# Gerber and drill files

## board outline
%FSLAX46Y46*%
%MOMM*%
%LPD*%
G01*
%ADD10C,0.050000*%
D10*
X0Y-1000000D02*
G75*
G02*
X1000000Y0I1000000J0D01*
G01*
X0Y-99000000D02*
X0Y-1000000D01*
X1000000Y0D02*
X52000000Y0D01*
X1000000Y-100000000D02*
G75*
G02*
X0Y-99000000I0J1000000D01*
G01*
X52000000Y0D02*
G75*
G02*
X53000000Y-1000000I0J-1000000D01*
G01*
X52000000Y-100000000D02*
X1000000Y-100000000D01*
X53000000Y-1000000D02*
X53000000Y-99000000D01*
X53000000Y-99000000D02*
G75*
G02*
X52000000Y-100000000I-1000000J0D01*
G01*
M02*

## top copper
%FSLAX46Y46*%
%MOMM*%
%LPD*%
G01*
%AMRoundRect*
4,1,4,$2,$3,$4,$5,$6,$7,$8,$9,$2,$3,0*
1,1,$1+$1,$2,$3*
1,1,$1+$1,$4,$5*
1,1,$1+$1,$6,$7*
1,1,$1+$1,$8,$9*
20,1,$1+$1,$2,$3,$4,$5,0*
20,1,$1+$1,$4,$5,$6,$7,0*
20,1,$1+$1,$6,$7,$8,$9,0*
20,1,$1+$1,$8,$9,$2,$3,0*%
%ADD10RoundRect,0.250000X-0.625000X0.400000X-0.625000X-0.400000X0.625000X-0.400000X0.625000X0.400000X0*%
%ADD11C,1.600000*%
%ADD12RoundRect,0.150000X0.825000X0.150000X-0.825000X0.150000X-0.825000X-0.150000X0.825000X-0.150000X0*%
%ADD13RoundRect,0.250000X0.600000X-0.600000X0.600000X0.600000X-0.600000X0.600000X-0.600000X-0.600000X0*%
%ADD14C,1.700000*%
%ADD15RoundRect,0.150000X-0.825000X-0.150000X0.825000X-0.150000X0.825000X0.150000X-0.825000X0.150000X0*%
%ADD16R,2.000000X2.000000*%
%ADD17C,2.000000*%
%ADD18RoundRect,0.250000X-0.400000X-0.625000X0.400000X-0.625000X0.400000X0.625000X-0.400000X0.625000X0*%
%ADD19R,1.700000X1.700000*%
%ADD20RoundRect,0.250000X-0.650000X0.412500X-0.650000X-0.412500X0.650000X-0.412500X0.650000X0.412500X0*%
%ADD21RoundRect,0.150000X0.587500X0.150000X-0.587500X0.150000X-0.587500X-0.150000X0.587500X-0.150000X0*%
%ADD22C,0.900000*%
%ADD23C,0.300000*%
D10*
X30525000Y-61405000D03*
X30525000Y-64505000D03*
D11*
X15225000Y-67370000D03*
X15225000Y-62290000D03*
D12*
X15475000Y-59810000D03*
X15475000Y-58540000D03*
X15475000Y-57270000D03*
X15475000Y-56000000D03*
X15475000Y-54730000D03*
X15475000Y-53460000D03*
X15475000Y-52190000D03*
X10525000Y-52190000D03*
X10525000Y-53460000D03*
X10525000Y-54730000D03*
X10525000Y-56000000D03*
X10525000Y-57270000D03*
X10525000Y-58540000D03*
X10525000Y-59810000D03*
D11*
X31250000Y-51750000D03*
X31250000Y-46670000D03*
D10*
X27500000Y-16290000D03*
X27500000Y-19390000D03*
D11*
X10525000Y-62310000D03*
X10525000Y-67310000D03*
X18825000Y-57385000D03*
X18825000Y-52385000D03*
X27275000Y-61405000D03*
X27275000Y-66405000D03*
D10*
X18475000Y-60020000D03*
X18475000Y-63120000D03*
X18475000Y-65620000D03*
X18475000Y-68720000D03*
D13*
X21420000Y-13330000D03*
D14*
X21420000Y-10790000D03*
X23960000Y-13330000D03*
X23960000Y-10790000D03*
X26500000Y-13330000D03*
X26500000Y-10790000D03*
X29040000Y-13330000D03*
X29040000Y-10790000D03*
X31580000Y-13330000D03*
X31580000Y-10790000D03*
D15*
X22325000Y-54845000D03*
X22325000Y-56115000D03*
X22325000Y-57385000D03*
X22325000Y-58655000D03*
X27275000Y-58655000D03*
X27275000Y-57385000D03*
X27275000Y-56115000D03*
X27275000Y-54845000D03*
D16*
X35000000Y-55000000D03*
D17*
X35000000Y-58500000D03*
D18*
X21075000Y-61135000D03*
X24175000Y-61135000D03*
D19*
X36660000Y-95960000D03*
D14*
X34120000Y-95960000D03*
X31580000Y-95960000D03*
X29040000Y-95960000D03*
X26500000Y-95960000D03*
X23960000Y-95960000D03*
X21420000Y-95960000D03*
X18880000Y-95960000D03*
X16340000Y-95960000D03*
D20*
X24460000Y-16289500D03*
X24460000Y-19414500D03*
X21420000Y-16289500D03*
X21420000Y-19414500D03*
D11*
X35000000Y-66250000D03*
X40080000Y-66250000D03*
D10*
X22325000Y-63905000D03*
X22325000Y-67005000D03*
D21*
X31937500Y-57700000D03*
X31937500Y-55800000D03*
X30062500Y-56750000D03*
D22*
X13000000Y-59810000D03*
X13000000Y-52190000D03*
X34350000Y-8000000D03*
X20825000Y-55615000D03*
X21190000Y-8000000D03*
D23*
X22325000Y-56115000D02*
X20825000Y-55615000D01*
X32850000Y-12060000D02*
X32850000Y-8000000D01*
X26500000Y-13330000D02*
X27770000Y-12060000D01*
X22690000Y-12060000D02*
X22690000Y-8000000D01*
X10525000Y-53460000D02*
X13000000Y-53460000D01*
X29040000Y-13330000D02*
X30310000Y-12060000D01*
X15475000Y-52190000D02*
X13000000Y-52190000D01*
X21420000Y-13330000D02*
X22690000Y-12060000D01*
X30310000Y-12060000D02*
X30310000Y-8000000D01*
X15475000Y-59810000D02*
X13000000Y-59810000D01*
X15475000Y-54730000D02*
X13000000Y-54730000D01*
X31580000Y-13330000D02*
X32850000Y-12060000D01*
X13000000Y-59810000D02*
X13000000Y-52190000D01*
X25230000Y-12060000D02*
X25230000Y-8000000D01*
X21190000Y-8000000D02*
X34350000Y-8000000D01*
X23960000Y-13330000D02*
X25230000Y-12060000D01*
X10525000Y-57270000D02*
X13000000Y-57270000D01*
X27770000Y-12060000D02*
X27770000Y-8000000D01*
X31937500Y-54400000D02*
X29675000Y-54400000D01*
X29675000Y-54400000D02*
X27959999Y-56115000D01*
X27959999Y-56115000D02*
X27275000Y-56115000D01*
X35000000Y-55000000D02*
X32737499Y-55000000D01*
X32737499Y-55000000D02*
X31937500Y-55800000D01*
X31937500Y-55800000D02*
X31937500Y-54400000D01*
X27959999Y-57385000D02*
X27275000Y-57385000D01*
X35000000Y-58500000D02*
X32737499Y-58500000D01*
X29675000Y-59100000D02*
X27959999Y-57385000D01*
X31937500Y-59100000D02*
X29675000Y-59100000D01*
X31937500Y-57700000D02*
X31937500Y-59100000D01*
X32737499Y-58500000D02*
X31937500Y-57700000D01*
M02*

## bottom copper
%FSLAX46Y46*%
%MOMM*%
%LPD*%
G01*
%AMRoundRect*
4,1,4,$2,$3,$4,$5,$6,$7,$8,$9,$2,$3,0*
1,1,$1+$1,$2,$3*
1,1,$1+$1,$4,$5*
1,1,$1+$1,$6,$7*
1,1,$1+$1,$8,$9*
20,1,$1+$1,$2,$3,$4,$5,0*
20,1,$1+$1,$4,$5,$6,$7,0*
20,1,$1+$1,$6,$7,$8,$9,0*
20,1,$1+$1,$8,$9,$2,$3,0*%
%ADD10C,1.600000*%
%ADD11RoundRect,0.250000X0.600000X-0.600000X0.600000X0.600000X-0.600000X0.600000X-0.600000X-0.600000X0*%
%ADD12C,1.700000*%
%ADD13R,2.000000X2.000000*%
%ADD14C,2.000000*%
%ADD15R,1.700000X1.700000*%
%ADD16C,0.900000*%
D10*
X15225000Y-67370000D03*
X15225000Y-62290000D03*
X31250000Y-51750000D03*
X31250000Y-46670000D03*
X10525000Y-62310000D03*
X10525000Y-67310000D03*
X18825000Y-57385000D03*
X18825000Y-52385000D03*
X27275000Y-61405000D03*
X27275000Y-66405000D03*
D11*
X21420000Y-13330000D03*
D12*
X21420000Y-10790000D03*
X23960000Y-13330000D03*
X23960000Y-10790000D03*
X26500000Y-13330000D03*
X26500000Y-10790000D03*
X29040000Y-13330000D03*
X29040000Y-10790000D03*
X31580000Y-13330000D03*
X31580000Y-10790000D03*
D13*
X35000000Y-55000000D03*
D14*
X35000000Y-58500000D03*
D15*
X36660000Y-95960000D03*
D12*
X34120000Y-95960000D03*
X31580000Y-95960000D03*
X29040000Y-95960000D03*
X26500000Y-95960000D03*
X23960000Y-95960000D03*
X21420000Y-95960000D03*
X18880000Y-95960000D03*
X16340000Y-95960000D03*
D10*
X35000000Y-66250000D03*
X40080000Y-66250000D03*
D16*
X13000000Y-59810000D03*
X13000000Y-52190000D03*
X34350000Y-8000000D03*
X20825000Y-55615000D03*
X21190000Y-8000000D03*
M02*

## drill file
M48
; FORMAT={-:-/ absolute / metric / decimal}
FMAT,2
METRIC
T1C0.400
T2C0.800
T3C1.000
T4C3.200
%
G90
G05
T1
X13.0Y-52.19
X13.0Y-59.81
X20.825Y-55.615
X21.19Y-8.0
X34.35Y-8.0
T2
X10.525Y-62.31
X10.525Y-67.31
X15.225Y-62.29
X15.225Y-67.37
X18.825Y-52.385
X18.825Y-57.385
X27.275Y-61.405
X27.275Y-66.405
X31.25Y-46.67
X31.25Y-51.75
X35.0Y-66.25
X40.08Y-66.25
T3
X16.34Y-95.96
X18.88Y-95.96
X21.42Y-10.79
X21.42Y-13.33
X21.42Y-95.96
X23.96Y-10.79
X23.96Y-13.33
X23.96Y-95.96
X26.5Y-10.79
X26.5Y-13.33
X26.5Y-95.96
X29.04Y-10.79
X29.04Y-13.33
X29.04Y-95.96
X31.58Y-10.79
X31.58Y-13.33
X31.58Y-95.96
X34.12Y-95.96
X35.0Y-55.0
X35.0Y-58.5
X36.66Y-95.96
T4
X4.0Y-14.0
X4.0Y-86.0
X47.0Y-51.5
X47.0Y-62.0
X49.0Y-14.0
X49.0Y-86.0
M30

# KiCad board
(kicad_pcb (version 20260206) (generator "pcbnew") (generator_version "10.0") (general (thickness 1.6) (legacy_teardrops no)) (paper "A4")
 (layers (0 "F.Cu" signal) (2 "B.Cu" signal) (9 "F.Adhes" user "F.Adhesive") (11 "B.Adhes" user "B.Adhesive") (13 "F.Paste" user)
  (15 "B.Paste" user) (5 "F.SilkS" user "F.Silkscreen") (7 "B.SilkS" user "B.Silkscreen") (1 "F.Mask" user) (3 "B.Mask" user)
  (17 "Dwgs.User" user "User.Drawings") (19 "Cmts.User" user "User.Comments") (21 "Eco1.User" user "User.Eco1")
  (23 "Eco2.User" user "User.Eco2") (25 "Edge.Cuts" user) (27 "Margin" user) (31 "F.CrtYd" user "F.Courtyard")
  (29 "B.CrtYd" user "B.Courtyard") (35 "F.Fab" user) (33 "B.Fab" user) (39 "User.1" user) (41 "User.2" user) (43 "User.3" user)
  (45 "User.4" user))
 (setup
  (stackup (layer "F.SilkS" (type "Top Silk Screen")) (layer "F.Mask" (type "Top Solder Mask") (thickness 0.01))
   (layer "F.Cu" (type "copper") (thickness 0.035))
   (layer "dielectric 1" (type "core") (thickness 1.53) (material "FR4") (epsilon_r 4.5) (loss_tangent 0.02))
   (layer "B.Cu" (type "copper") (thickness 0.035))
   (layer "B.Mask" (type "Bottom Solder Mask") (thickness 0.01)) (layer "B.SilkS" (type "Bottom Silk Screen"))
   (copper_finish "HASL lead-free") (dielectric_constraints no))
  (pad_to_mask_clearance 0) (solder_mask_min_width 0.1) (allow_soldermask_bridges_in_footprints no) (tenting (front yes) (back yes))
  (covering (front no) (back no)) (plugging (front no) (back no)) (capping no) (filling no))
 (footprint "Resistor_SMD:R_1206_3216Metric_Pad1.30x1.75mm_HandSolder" (layer "F.Cu") (at 30.525 62.955 -90)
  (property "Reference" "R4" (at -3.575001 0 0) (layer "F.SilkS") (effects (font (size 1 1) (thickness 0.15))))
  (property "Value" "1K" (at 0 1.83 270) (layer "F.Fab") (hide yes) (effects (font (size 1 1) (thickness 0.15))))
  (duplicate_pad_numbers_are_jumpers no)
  (pad "1" smd roundrect (at -1.55 0 270) (size 1.3 1.75) (layers "F.Cu" "F.Mask" "F.Paste") (roundrect_rratio 0.192308) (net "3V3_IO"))
  (pad "2" smd roundrect (at 1.55 0 270) (size 1.3 1.75) (layers "F.Cu" "F.Mask" "F.Paste") (roundrect_rratio 0.192308)
   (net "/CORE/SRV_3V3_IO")))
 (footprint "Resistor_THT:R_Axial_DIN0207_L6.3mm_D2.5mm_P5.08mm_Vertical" (layer "F.Cu") (at 15.225 67.37 90)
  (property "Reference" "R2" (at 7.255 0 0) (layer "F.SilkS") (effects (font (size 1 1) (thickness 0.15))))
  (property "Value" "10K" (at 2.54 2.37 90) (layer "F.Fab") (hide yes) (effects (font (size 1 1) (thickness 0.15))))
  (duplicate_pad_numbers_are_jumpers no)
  (pad "1" thru_hole circle (at 0 0 90) (size 1.6 1.6) (drill 0.8) (layers "*.Cu" "*.Mask") (remove_unused_layers no) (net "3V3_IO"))
  (pad "2" thru_hole circle (at 5.08 0 90) (size 1.6 1.6) (drill 0.8) (layers "*.Cu" "*.Mask") (remove_unused_layers no) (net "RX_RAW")))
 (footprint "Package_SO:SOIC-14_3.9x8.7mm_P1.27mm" (layer "F.Cu") (at 13 56 180)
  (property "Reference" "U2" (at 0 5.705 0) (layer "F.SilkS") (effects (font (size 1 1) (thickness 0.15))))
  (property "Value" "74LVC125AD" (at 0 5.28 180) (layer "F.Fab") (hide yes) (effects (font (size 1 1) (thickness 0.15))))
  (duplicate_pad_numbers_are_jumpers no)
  (pad "1" smd roundrect (at -2.475 -3.81 180) (size 1.95 0.6) (layers "F.Cu" "F.Mask" "F.Paste") (roundrect_rratio 0.25) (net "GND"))
  (pad "2" smd roundrect (at -2.475 -2.54 180) (size 1.95 0.6) (layers "F.Cu" "F.Mask" "F.Paste") (roundrect_rratio 0.25) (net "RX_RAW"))
  (pad "3" smd roundrect (at -2.475 -1.27 180) (size 1.95 0.6) (layers "F.Cu" "F.Mask" "F.Paste") (roundrect_rratio 0.25)
   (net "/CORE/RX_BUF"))
  (pad "4" smd roundrect (at -2.475 0 180) (size 1.95 0.6) (layers "F.Cu" "F.Mask" "F.Paste") (roundrect_rratio 0.25) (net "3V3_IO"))
  (pad "5" smd roundrect (at -2.475 1.27 180) (size 1.95 0.6) (layers "F.Cu" "F.Mask" "F.Paste") (roundrect_rratio 0.25) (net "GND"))
  (pad "6" smd roundrect (at -2.475 2.54 180) (size 1.95 0.6) (layers "F.Cu" "F.Mask" "F.Paste") (roundrect_rratio 0.25)
   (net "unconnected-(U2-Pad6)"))
  (pad "7" smd roundrect (at -2.475 3.81 180) (size 1.95 0.6) (layers "F.Cu" "F.Mask" "F.Paste") (roundrect_rratio 0.25) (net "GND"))
  (pad "8" smd roundrect (at 2.475 3.81 180) (size 1.95 0.6) (layers "F.Cu" "F.Mask" "F.Paste") (roundrect_rratio 0.25)
   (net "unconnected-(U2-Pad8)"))
  (pad "9" smd roundrect (at 2.475 2.54 180) (size 1.95 0.6) (layers "F.Cu" "F.Mask" "F.Paste") (roundrect_rratio 0.25) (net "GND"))
  (pad "10" smd roundrect (at 2.475 1.27 180) (size 1.95 0.6) (layers "F.Cu" "F.Mask" "F.Paste") (roundrect_rratio 0.25) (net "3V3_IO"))
  (pad "11" smd roundrect (at 2.475 0 180) (size 1.95 0.6) (layers "F.Cu" "F.Mask" "F.Paste") (roundrect_rratio 0.25)
   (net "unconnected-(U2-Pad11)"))
  (pad "12" smd roundrect (at 2.475 -1.27 180) (size 1.95 0.6) (layers "F.Cu" "F.Mask" "F.Paste") (roundrect_rratio 0.25) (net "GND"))
  (pad "13" smd roundrect (at 2.475 -2.54 180) (size 1.95 0.6) (layers "F.Cu" "F.Mask" "F.Paste") (roundrect_rratio 0.25) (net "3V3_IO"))
  (pad "14" smd roundrect (at 2.475 -3.81 180) (size 1.95 0.6) (layers "F.Cu" "F.Mask" "F.Paste") (roundrect_rratio 0.25) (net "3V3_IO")))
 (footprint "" (layer "F.Cu") (at 49 14)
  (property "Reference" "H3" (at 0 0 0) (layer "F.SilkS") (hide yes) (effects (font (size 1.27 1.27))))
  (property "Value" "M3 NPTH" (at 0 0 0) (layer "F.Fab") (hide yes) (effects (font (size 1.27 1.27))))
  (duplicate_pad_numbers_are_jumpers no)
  (pad "" np_thru_hole circle (at 0 0) (size 3.2 3.2) (drill 3.2) (layers "*.Cu")))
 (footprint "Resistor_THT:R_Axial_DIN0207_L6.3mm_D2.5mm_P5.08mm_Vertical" (layer "F.Cu") (at 31.25 51.75 90)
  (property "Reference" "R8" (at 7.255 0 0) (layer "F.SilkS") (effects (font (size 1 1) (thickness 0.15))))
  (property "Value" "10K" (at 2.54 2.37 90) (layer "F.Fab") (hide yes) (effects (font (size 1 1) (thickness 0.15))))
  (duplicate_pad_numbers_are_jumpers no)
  (pad "1" thru_hole circle (at 0 0 90) (size 1.6 1.6) (drill 0.8) (layers "*.Cu" "*.Mask") (remove_unused_layers no) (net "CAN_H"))
  (pad "2" thru_hole circle (at 5.08 0 90) (size 1.6 1.6) (drill 0.8) (layers "*.Cu" "*.Mask") (remove_unused_layers no)
   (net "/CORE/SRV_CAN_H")))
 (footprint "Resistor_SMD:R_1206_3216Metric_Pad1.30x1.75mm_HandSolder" (layer "F.Cu") (at 27.5 17.84 -90)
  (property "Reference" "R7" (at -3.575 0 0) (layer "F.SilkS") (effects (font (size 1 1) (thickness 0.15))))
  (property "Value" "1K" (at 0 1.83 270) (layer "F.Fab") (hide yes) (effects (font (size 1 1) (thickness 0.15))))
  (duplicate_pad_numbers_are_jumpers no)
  (pad "1" smd roundrect (at -1.55 0 270) (size 1.3 1.75) (layers "F.Cu" "F.Mask" "F.Paste") (roundrect_rratio 0.192308)
   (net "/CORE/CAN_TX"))
  (pad "2" smd roundrect (at 1.55 0 270) (size 1.3 1.75) (layers "F.Cu" "F.Mask" "F.Paste") (roundrect_rratio 0.192308)
   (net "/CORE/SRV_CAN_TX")))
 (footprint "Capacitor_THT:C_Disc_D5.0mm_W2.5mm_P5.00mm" (layer "F.Cu") (at 10.525 62.31 -90)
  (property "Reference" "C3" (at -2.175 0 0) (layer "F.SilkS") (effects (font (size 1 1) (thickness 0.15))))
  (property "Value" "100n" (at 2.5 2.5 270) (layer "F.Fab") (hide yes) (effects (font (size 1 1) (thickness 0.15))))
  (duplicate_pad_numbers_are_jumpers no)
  (pad "1" thru_hole circle (at 0 0 270) (size 1.6 1.6) (drill 0.8) (layers "*.Cu" "*.Mask") (remove_unused_layers no) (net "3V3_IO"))
  (pad "2" thru_hole circle (at 5 0 270) (size 1.6 1.6) (drill 0.8) (layers "*.Cu" "*.Mask") (remove_unused_layers no) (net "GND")))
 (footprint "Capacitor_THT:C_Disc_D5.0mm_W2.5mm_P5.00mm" (layer "F.Cu") (at 18.825 57.385 90)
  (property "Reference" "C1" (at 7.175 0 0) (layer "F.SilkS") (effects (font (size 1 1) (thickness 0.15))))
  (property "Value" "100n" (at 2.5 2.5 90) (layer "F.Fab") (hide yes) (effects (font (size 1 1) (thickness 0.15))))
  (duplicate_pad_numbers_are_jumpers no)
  (pad "1" thru_hole circle (at 0 0 90) (size 1.6 1.6) (drill 0.8) (layers "*.Cu" "*.Mask") (remove_unused_layers no) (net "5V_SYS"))
  (pad "2" thru_hole circle (at 5 0 90) (size 1.6 1.6) (drill 0.8) (layers "*.Cu" "*.Mask") (remove_unused_layers no) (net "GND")))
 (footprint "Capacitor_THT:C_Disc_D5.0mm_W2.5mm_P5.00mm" (layer "F.Cu") (at 27.275 61.405 -90)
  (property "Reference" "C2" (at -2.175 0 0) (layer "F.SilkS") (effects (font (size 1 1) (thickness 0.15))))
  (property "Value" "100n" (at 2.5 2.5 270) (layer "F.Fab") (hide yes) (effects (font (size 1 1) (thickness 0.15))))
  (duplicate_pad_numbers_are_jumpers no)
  (pad "1" thru_hole circle (at 0 0 270) (size 1.6 1.6) (drill 0.8) (layers "*.Cu" "*.Mask") (remove_unused_layers no) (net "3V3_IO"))
  (pad "2" thru_hole circle (at 5 0 270) (size 1.6 1.6) (drill 0.8) (layers "*.Cu" "*.Mask") (remove_unused_layers no) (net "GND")))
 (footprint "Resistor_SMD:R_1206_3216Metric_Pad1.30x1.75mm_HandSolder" (layer "F.Cu") (at 18.475 61.57 -90)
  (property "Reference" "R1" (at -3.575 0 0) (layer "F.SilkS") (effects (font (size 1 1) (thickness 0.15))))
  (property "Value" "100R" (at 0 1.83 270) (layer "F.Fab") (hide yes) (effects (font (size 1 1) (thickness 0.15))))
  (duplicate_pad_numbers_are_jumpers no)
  (pad "1" smd roundrect (at -1.55 0 270) (size 1.3 1.75) (layers "F.Cu" "F.Mask" "F.Paste") (roundrect_rratio 0.192308)
   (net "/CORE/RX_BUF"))
  (pad "2" smd roundrect (at 1.55 0 270) (size 1.3 1.75) (layers "F.Cu" "F.Mask" "F.Paste") (roundrect_rratio 0.192308) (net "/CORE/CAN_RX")))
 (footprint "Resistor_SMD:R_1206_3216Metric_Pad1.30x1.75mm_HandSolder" (layer "F.Cu") (at 18.475 67.17 -90)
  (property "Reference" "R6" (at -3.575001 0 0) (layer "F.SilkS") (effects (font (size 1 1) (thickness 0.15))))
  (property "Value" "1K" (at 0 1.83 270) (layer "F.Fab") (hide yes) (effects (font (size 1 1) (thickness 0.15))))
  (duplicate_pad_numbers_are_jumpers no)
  (pad "1" smd roundrect (at -1.55 0 270) (size 1.3 1.75) (layers "F.Cu" "F.Mask" "F.Paste") (roundrect_rratio 0.192308)
   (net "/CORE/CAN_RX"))
  (pad "2" smd roundrect (at 1.55 0 270) (size 1.3 1.75) (layers "F.Cu" "F.Mask" "F.Paste") (roundrect_rratio 0.192308)
   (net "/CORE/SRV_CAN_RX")))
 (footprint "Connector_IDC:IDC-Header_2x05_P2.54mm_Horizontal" (layer "F.Cu") (at 21.42 13.33 90)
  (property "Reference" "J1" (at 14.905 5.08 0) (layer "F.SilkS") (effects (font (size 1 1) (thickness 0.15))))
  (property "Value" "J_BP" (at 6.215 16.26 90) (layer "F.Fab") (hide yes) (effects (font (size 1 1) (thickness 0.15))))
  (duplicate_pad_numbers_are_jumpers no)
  (pad "1" thru_hole roundrect (at 0 0 90) (size 1.7 1.7) (drill 1) (layers "*.Cu" "*.Mask") (remove_unused_layers no)
   (roundrect_rratio 0.147059) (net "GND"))
  (pad "2" thru_hole circle (at 2.54 0 90) (size 1.7 1.7) (drill 1) (layers "*.Cu" "*.Mask") (remove_unused_layers no) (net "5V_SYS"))
  (pad "3" thru_hole circle (at 0 2.54 90) (size 1.7 1.7) (drill 1) (layers "*.Cu" "*.Mask") (remove_unused_layers no) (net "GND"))
  (pad "4" thru_hole circle (at 2.54 2.54 90) (size 1.7 1.7) (drill 1) (layers "*.Cu" "*.Mask") (remove_unused_layers no) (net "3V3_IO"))
  (pad "5" thru_hole circle (at 0 5.08 90) (size 1.7 1.7) (drill 1) (layers "*.Cu" "*.Mask") (remove_unused_layers no) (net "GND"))
  (pad "6" thru_hole circle (at 2.54 5.08 90) (size 1.7 1.7) (drill 1) (layers "*.Cu" "*.Mask") (remove_unused_layers no)
   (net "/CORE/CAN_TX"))
  (pad "7" thru_hole circle (at 0 7.62 90) (size 1.7 1.7) (drill 1) (layers "*.Cu" "*.Mask") (remove_unused_layers no) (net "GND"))
  (pad "8" thru_hole circle (at 2.54 7.62 90) (size 1.7 1.7) (drill 1) (layers "*.Cu" "*.Mask") (remove_unused_layers no)
   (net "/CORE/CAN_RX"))
  (pad "9" thru_hole circle (at 0 10.16 90) (size 1.7 1.7) (drill 1) (layers "*.Cu" "*.Mask") (remove_unused_layers no) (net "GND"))
  (pad "10" thru_hole circle (at 2.54 10.16 90) (size 1.7 1.7) (drill 1) (layers "*.Cu" "*.Mask") (remove_unused_layers no) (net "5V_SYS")))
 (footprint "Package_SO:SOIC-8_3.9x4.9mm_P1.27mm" (layer "F.Cu") (at 24.8 56.75)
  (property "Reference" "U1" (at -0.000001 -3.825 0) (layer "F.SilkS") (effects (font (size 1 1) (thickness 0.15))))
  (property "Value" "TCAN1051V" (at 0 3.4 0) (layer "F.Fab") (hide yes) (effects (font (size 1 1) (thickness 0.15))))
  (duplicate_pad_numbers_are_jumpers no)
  (pad "1" smd roundrect (at -2.475 -1.905) (size 1.95 0.6) (layers "F.Cu" "F.Mask" "F.Paste") (roundrect_rratio 0.25) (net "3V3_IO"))
  (pad "2" smd roundrect (at -2.475 -0.635) (size 1.95 0.6) (layers "F.Cu" "F.Mask" "F.Paste") (roundrect_rratio 0.25) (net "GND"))
  (pad "3" smd roundrect (at -2.475 0.635) (size 1.95 0.6) (layers "F.Cu" "F.Mask" "F.Paste") (roundrect_rratio 0.25) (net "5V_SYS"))
  (pad "4" smd roundrect (at -2.475 1.905) (size 1.95 0.6) (layers "F.Cu" "F.Mask" "F.Paste") (roundrect_rratio 0.25) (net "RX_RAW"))
  (pad "5" smd roundrect (at 2.475 1.905) (size 1.95 0.6) (layers "F.Cu" "F.Mask" "F.Paste") (roundrect_rratio 0.25) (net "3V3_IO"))
  (pad "6" smd roundrect (at 2.475 0.635) (size 1.95 0.6) (layers "F.Cu" "F.Mask" "F.Paste") (roundrect_rratio 0.25) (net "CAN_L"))
  (pad "7" smd roundrect (at 2.475 -0.635) (size 1.95 0.6) (layers "F.Cu" "F.Mask" "F.Paste") (roundrect_rratio 0.25) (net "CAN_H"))
  (pad "8" smd roundrect (at 2.475 -1.905) (size 1.95 0.6) (layers "F.Cu" "F.Mask" "F.Paste") (roundrect_rratio 0.25) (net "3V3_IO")))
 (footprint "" (layer "F.Cu") (at 49 86)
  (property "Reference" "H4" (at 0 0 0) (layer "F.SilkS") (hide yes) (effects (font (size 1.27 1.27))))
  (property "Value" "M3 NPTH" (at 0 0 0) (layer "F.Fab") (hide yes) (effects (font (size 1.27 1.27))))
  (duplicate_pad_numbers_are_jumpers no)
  (pad "" np_thru_hole circle (at 0 0) (size 3.2 3.2) (drill 3.2) (layers "*.Cu")))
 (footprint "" (layer "F.Cu") (at 4 86)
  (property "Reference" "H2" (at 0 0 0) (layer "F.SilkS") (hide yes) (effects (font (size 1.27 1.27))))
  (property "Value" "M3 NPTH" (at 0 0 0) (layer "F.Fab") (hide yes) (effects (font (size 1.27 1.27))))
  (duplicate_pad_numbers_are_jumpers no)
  (pad "" np_thru_hole circle (at 0 0) (size 3.2 3.2) (drill 3.2) (layers "*.Cu")))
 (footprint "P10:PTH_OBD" (layer "F.Cu") (at 35 55 -90)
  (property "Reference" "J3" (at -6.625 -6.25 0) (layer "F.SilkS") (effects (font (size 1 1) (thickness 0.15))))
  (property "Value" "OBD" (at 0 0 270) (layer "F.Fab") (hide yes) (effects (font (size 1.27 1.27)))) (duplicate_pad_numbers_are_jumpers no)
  (pad "" np_thru_hole circle (at -3.5 -12 270) (size 3.2 3.2) (drill 3.2) (layers "*.Cu" "*.Mask"))
  (pad "" np_thru_hole circle (at 7 -12 270) (size 3.2 3.2) (drill 3.2) (layers "*.Cu" "*.Mask"))
  (pad "1" thru_hole rect (at 0 0 270) (size 2 2) (drill 1) (layers "*.Cu" "*.Mask") (remove_unused_layers no) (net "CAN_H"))
  (pad "2" thru_hole circle (at 3.5 0 270) (size 2 2) (drill 1) (layers "*.Cu" "*.Mask") (remove_unused_layers no) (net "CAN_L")))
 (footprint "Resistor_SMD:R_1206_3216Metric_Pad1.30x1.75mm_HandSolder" (layer "F.Cu") (at 22.625 61.135)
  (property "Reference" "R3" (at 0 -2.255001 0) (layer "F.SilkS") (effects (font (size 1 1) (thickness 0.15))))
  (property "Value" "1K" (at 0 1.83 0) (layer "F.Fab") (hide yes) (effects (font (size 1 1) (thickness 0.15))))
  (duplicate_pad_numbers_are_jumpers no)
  (pad "1" smd roundrect (at -1.55 0) (size 1.3 1.75) (layers "F.Cu" "F.Mask" "F.Paste") (roundrect_rratio 0.192308) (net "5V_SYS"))
  (pad "2" smd roundrect (at 1.55 0) (size 1.3 1.75) (layers "F.Cu" "F.Mask" "F.Paste") (roundrect_rratio 0.192308) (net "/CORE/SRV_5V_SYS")))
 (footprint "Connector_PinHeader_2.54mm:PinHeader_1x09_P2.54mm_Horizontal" (layer "F.Cu") (at 36.66 95.96 -90)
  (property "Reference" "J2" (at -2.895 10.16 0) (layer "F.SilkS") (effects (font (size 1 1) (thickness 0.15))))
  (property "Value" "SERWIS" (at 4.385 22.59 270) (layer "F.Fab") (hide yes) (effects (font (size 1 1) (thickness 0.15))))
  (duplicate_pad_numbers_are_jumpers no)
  (pad "1" thru_hole rect (at 0 0 270) (size 1.7 1.7) (drill 1) (layers "*.Cu" "*.Mask") (remove_unused_layers no) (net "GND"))
  (pad "2" thru_hole circle (at 0 2.54 270) (size 1.7 1.7) (drill 1) (layers "*.Cu" "*.Mask") (remove_unused_layers no)
   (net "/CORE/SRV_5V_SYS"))
  (pad "3" thru_hole circle (at 0 5.08 270) (size 1.7 1.7) (drill 1) (layers "*.Cu" "*.Mask") (remove_unused_layers no)
   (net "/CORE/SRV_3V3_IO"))
  (pad "4" thru_hole circle (at 0 7.62 270) (size 1.7 1.7) (drill 1) (layers "*.Cu" "*.Mask") (remove_unused_layers no)
   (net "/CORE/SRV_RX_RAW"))
  (pad "5" thru_hole circle (at 0 10.16 270) (size 1.7 1.7) (drill 1) (layers "*.Cu" "*.Mask") (remove_unused_layers no)
   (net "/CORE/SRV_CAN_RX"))
  (pad "6" thru_hole circle (at 0 12.7 270) (size 1.7 1.7) (drill 1) (layers "*.Cu" "*.Mask") (remove_unused_layers no)
   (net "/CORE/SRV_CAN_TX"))
  (pad "7" thru_hole circle (at 0 15.24 270) (size 1.7 1.7) (drill 1) (layers "*.Cu" "*.Mask") (remove_unused_layers no)
   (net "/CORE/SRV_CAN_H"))
  (pad "8" thru_hole circle (at 0 17.78 270) (size 1.7 1.7) (drill 1) (layers "*.Cu" "*.Mask") (remove_unused_layers no)
   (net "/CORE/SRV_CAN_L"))
  (pad "9" thru_hole circle (at 0 20.32 270) (size 1.7 1.7) (drill 1) (layers "*.Cu" "*.Mask") (remove_unused_layers no) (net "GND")))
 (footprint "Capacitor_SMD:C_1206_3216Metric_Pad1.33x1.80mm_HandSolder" (layer "F.Cu") (at 24.46 17.852 -90)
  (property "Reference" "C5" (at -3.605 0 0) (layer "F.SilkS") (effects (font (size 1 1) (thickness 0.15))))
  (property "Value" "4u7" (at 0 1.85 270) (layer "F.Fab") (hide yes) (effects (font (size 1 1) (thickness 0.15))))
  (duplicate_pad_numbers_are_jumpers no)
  (pad "1" smd roundrect (at -1.5625 0 270) (size 1.325 1.8) (layers "F.Cu" "F.Mask" "F.Paste") (roundrect_rratio 0.188679) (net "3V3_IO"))
  (pad "2" smd roundrect (at 1.5625 0 270) (size 1.325 1.8) (layers "F.Cu" "F.Mask" "F.Paste") (roundrect_rratio 0.188679) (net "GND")))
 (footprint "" (layer "F.Cu") (at 4 14)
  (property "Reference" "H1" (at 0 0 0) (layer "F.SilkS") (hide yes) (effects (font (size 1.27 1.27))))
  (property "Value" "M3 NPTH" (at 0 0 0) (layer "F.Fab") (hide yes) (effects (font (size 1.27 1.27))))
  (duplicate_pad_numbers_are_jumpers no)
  (pad "" np_thru_hole circle (at 0 0) (size 3.2 3.2) (drill 3.2) (layers "*.Cu")))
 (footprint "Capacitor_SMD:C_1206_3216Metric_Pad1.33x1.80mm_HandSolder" (layer "F.Cu") (at 21.42 17.852 -90)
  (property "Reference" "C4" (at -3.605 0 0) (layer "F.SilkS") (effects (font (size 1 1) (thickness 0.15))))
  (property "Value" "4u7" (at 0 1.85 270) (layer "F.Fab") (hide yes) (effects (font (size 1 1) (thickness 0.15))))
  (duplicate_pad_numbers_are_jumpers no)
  (pad "1" smd roundrect (at -1.5625 0 270) (size 1.325 1.8) (layers "F.Cu" "F.Mask" "F.Paste") (roundrect_rratio 0.188679) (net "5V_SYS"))
  (pad "2" smd roundrect (at 1.5625 0 270) (size 1.325 1.8) (layers "F.Cu" "F.Mask" "F.Paste") (roundrect_rratio 0.188679) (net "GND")))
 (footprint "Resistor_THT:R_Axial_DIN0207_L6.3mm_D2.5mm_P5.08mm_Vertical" (layer "F.Cu") (at 35 66.25)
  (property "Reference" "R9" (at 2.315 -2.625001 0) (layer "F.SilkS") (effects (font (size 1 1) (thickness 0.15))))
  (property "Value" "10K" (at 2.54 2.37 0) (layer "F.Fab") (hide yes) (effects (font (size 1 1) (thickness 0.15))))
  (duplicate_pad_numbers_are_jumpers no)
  (pad "1" thru_hole circle (at 0 0) (size 1.6 1.6) (drill 0.8) (layers "*.Cu" "*.Mask") (remove_unused_layers no) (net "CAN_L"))
  (pad "2" thru_hole circle (at 5.08 0) (size 1.6 1.6) (drill 0.8) (layers "*.Cu" "*.Mask") (remove_unused_layers no)
   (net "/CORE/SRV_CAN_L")))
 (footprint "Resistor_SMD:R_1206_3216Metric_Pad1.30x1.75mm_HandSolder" (layer "F.Cu") (at 22.325 65.455 -90)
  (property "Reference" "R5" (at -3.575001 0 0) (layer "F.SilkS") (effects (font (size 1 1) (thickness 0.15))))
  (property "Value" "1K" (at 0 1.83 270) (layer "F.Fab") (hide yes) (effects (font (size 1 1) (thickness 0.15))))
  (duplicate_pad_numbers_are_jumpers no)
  (pad "1" smd roundrect (at -1.55 0 270) (size 1.3 1.75) (layers "F.Cu" "F.Mask" "F.Paste") (roundrect_rratio 0.192308) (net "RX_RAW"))
  (pad "2" smd roundrect (at 1.55 0 270) (size 1.3 1.75) (layers "F.Cu" "F.Mask" "F.Paste") (roundrect_rratio 0.192308)
   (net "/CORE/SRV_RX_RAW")))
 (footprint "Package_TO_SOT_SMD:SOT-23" (layer "F.Cu") (at 31 56.75 180)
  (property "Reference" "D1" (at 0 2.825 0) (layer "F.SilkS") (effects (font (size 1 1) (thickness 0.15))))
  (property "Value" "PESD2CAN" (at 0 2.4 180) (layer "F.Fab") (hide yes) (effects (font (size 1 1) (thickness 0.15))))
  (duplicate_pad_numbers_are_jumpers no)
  (pad "1" smd roundrect (at -0.9375 -0.95 180) (size 1.475 0.6) (layers "F.Cu" "F.Mask" "F.Paste") (roundrect_rratio 0.25) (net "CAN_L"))
  (pad "2" smd roundrect (at -0.9375 0.95 180) (size 1.475 0.6) (layers "F.Cu" "F.Mask" "F.Paste") (roundrect_rratio 0.25) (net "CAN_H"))
  (pad "3" smd roundrect (at 0.9375 0 180) (size 1.475 0.6) (layers "F.Cu" "F.Mask" "F.Paste") (roundrect_rratio 0.25) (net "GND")))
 (gr_arc (start 0 1) (mid 0.292893 0.292893) (end 1 0) (stroke (width 0.05) (type default)) (layer "Edge.Cuts"))
 (gr_line (start 0 99) (end 0 1) (stroke (width 0.05) (type default)) (layer "Edge.Cuts"))
 (gr_line (start 1 0) (end 52 0) (stroke (width 0.05) (type default)) (layer "Edge.Cuts"))
 (gr_arc (start 1 100) (mid 0.292893 99.707107) (end 0 99) (stroke (width 0.05) (type default)) (layer "Edge.Cuts"))
 (gr_arc (start 52 0) (mid 52.707107 0.292893) (end 53 1) (stroke (width 0.05) (type default)) (layer "Edge.Cuts"))
 (gr_line (start 52 100) (end 1 100) (stroke (width 0.05) (type default)) (layer "Edge.Cuts"))
 (gr_line (start 53 1) (end 53 99) (stroke (width 0.05) (type default)) (layer "Edge.Cuts"))
 (gr_arc (start 53 99) (mid 52.707107 99.707107) (end 52 100) (stroke (width 0.05) (type default)) (layer "Edge.Cuts"))
 (segment (start 22.325 56.115) (end 20.825 55.615) (width 0.3) (locked yes) (layer "F.Cu") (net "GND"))
 (segment (start 32.85 12.06) (end 32.85 8) (width 0.3) (locked yes) (layer "F.Cu") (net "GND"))
 (segment (start 26.5 13.33) (end 27.77 12.06) (width 0.3) (locked yes) (layer "F.Cu") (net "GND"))
 (segment (start 22.69 12.06) (end 22.69 8) (width 0.3) (locked yes) (layer "F.Cu") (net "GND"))
 (segment (start 10.525 53.46) (end 13 53.46) (width 0.3) (locked yes) (layer "F.Cu") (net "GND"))
 (segment (start 29.04 13.33) (end 30.31 12.06) (width 0.3) (locked yes) (layer "F.Cu") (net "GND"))
 (segment (start 15.475 52.19) (end 13 52.19) (width 0.3) (locked yes) (layer "F.Cu") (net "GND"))
 (segment (start 21.42 13.33) (end 22.69 12.06) (width 0.3) (locked yes) (layer "F.Cu") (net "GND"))
 (segment (start 30.31 12.06) (end 30.31 8) (width 0.3) (locked yes) (layer "F.Cu") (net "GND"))
 (segment (start 15.475 59.81) (end 13 59.81) (width 0.3) (locked yes) (layer "F.Cu") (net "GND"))
 (segment (start 15.475 54.73) (end 13 54.73) (width 0.3) (locked yes) (layer "F.Cu") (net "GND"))
 (segment (start 31.58 13.33) (end 32.85 12.06) (width 0.3) (locked yes) (layer "F.Cu") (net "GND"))
 (segment (start 13 59.81) (end 13 52.19) (width 0.3) (locked yes) (layer "F.Cu") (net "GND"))
 (segment (start 25.23 12.06) (end 25.23 8) (width 0.3) (locked yes) (layer "F.Cu") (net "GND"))
 (segment (start 21.19 8) (end 34.35 8) (width 0.3) (locked yes) (layer "F.Cu") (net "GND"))
 (segment (start 23.96 13.33) (end 25.23 12.06) (width 0.3) (locked yes) (layer "F.Cu") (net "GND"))
 (segment (start 10.525 57.27) (end 13 57.27) (width 0.3) (locked yes) (layer "F.Cu") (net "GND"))
 (segment (start 27.77 12.06) (end 27.77 8) (width 0.3) (locked yes) (layer "F.Cu") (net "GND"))
 (via (at 13 59.81) (size 0.9) (drill 0.4) (layers "F.Cu" "B.Cu") (locked yes) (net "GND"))
 (via (at 13 52.19) (size 0.9) (drill 0.4) (layers "F.Cu" "B.Cu") (locked yes) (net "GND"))
 (via (at 34.35 8) (size 0.9) (drill 0.4) (layers "F.Cu" "B.Cu") (locked yes) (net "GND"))
 (via (at 20.825 55.615) (size 0.9) (drill 0.4) (layers "F.Cu" "B.Cu") (locked yes) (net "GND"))
 (via (at 21.19 8) (size 0.9) (drill 0.4) (layers "F.Cu" "B.Cu") (locked yes) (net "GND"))
 (segment (start 31.9375 54.4) (end 29.675 54.4) (width 0.3) (locked yes) (layer "F.Cu") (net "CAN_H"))
 (segment (start 29.675 54.4) (end 27.959999 56.115) (width 0.3) (locked yes) (layer "F.Cu") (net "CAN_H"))
 (segment (start 27.959999 56.115) (end 27.275 56.115) (width 0.3) (locked yes) (layer "F.Cu") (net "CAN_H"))
 (segment (start 35 55) (end 32.737499 55) (width 0.3) (locked yes) (layer "F.Cu") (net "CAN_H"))
 (segment (start 32.737499 55) (end 31.9375 55.8) (width 0.3) (locked yes) (layer "F.Cu") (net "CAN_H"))
 (segment (start 31.9375 55.8) (end 31.9375 54.4) (width 0.3) (locked yes) (layer "F.Cu") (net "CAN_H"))
 (segment (start 27.959999 57.385) (end 27.275 57.385) (width 0.3) (locked yes) (layer "F.Cu") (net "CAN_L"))
 (segment (start 35 58.5) (end 32.737499 58.5) (width 0.3) (locked yes) (layer "F.Cu") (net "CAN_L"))
 (segment (start 29.675 59.1) (end 27.959999 57.385) (width 0.3) (locked yes) (layer "F.Cu") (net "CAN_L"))
 (segment (start 31.9375 59.1) (end 29.675 59.1) (width 0.3) (locked yes) (layer "F.Cu") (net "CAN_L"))
 (segment (start 31.9375 57.7) (end 31.9375 59.1) (width 0.3) (locked yes) (layer "F.Cu") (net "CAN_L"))
 (segment (start 32.737499 58.5) (end 31.9375 57.7) (width 0.3) (locked yes) (layer "F.Cu") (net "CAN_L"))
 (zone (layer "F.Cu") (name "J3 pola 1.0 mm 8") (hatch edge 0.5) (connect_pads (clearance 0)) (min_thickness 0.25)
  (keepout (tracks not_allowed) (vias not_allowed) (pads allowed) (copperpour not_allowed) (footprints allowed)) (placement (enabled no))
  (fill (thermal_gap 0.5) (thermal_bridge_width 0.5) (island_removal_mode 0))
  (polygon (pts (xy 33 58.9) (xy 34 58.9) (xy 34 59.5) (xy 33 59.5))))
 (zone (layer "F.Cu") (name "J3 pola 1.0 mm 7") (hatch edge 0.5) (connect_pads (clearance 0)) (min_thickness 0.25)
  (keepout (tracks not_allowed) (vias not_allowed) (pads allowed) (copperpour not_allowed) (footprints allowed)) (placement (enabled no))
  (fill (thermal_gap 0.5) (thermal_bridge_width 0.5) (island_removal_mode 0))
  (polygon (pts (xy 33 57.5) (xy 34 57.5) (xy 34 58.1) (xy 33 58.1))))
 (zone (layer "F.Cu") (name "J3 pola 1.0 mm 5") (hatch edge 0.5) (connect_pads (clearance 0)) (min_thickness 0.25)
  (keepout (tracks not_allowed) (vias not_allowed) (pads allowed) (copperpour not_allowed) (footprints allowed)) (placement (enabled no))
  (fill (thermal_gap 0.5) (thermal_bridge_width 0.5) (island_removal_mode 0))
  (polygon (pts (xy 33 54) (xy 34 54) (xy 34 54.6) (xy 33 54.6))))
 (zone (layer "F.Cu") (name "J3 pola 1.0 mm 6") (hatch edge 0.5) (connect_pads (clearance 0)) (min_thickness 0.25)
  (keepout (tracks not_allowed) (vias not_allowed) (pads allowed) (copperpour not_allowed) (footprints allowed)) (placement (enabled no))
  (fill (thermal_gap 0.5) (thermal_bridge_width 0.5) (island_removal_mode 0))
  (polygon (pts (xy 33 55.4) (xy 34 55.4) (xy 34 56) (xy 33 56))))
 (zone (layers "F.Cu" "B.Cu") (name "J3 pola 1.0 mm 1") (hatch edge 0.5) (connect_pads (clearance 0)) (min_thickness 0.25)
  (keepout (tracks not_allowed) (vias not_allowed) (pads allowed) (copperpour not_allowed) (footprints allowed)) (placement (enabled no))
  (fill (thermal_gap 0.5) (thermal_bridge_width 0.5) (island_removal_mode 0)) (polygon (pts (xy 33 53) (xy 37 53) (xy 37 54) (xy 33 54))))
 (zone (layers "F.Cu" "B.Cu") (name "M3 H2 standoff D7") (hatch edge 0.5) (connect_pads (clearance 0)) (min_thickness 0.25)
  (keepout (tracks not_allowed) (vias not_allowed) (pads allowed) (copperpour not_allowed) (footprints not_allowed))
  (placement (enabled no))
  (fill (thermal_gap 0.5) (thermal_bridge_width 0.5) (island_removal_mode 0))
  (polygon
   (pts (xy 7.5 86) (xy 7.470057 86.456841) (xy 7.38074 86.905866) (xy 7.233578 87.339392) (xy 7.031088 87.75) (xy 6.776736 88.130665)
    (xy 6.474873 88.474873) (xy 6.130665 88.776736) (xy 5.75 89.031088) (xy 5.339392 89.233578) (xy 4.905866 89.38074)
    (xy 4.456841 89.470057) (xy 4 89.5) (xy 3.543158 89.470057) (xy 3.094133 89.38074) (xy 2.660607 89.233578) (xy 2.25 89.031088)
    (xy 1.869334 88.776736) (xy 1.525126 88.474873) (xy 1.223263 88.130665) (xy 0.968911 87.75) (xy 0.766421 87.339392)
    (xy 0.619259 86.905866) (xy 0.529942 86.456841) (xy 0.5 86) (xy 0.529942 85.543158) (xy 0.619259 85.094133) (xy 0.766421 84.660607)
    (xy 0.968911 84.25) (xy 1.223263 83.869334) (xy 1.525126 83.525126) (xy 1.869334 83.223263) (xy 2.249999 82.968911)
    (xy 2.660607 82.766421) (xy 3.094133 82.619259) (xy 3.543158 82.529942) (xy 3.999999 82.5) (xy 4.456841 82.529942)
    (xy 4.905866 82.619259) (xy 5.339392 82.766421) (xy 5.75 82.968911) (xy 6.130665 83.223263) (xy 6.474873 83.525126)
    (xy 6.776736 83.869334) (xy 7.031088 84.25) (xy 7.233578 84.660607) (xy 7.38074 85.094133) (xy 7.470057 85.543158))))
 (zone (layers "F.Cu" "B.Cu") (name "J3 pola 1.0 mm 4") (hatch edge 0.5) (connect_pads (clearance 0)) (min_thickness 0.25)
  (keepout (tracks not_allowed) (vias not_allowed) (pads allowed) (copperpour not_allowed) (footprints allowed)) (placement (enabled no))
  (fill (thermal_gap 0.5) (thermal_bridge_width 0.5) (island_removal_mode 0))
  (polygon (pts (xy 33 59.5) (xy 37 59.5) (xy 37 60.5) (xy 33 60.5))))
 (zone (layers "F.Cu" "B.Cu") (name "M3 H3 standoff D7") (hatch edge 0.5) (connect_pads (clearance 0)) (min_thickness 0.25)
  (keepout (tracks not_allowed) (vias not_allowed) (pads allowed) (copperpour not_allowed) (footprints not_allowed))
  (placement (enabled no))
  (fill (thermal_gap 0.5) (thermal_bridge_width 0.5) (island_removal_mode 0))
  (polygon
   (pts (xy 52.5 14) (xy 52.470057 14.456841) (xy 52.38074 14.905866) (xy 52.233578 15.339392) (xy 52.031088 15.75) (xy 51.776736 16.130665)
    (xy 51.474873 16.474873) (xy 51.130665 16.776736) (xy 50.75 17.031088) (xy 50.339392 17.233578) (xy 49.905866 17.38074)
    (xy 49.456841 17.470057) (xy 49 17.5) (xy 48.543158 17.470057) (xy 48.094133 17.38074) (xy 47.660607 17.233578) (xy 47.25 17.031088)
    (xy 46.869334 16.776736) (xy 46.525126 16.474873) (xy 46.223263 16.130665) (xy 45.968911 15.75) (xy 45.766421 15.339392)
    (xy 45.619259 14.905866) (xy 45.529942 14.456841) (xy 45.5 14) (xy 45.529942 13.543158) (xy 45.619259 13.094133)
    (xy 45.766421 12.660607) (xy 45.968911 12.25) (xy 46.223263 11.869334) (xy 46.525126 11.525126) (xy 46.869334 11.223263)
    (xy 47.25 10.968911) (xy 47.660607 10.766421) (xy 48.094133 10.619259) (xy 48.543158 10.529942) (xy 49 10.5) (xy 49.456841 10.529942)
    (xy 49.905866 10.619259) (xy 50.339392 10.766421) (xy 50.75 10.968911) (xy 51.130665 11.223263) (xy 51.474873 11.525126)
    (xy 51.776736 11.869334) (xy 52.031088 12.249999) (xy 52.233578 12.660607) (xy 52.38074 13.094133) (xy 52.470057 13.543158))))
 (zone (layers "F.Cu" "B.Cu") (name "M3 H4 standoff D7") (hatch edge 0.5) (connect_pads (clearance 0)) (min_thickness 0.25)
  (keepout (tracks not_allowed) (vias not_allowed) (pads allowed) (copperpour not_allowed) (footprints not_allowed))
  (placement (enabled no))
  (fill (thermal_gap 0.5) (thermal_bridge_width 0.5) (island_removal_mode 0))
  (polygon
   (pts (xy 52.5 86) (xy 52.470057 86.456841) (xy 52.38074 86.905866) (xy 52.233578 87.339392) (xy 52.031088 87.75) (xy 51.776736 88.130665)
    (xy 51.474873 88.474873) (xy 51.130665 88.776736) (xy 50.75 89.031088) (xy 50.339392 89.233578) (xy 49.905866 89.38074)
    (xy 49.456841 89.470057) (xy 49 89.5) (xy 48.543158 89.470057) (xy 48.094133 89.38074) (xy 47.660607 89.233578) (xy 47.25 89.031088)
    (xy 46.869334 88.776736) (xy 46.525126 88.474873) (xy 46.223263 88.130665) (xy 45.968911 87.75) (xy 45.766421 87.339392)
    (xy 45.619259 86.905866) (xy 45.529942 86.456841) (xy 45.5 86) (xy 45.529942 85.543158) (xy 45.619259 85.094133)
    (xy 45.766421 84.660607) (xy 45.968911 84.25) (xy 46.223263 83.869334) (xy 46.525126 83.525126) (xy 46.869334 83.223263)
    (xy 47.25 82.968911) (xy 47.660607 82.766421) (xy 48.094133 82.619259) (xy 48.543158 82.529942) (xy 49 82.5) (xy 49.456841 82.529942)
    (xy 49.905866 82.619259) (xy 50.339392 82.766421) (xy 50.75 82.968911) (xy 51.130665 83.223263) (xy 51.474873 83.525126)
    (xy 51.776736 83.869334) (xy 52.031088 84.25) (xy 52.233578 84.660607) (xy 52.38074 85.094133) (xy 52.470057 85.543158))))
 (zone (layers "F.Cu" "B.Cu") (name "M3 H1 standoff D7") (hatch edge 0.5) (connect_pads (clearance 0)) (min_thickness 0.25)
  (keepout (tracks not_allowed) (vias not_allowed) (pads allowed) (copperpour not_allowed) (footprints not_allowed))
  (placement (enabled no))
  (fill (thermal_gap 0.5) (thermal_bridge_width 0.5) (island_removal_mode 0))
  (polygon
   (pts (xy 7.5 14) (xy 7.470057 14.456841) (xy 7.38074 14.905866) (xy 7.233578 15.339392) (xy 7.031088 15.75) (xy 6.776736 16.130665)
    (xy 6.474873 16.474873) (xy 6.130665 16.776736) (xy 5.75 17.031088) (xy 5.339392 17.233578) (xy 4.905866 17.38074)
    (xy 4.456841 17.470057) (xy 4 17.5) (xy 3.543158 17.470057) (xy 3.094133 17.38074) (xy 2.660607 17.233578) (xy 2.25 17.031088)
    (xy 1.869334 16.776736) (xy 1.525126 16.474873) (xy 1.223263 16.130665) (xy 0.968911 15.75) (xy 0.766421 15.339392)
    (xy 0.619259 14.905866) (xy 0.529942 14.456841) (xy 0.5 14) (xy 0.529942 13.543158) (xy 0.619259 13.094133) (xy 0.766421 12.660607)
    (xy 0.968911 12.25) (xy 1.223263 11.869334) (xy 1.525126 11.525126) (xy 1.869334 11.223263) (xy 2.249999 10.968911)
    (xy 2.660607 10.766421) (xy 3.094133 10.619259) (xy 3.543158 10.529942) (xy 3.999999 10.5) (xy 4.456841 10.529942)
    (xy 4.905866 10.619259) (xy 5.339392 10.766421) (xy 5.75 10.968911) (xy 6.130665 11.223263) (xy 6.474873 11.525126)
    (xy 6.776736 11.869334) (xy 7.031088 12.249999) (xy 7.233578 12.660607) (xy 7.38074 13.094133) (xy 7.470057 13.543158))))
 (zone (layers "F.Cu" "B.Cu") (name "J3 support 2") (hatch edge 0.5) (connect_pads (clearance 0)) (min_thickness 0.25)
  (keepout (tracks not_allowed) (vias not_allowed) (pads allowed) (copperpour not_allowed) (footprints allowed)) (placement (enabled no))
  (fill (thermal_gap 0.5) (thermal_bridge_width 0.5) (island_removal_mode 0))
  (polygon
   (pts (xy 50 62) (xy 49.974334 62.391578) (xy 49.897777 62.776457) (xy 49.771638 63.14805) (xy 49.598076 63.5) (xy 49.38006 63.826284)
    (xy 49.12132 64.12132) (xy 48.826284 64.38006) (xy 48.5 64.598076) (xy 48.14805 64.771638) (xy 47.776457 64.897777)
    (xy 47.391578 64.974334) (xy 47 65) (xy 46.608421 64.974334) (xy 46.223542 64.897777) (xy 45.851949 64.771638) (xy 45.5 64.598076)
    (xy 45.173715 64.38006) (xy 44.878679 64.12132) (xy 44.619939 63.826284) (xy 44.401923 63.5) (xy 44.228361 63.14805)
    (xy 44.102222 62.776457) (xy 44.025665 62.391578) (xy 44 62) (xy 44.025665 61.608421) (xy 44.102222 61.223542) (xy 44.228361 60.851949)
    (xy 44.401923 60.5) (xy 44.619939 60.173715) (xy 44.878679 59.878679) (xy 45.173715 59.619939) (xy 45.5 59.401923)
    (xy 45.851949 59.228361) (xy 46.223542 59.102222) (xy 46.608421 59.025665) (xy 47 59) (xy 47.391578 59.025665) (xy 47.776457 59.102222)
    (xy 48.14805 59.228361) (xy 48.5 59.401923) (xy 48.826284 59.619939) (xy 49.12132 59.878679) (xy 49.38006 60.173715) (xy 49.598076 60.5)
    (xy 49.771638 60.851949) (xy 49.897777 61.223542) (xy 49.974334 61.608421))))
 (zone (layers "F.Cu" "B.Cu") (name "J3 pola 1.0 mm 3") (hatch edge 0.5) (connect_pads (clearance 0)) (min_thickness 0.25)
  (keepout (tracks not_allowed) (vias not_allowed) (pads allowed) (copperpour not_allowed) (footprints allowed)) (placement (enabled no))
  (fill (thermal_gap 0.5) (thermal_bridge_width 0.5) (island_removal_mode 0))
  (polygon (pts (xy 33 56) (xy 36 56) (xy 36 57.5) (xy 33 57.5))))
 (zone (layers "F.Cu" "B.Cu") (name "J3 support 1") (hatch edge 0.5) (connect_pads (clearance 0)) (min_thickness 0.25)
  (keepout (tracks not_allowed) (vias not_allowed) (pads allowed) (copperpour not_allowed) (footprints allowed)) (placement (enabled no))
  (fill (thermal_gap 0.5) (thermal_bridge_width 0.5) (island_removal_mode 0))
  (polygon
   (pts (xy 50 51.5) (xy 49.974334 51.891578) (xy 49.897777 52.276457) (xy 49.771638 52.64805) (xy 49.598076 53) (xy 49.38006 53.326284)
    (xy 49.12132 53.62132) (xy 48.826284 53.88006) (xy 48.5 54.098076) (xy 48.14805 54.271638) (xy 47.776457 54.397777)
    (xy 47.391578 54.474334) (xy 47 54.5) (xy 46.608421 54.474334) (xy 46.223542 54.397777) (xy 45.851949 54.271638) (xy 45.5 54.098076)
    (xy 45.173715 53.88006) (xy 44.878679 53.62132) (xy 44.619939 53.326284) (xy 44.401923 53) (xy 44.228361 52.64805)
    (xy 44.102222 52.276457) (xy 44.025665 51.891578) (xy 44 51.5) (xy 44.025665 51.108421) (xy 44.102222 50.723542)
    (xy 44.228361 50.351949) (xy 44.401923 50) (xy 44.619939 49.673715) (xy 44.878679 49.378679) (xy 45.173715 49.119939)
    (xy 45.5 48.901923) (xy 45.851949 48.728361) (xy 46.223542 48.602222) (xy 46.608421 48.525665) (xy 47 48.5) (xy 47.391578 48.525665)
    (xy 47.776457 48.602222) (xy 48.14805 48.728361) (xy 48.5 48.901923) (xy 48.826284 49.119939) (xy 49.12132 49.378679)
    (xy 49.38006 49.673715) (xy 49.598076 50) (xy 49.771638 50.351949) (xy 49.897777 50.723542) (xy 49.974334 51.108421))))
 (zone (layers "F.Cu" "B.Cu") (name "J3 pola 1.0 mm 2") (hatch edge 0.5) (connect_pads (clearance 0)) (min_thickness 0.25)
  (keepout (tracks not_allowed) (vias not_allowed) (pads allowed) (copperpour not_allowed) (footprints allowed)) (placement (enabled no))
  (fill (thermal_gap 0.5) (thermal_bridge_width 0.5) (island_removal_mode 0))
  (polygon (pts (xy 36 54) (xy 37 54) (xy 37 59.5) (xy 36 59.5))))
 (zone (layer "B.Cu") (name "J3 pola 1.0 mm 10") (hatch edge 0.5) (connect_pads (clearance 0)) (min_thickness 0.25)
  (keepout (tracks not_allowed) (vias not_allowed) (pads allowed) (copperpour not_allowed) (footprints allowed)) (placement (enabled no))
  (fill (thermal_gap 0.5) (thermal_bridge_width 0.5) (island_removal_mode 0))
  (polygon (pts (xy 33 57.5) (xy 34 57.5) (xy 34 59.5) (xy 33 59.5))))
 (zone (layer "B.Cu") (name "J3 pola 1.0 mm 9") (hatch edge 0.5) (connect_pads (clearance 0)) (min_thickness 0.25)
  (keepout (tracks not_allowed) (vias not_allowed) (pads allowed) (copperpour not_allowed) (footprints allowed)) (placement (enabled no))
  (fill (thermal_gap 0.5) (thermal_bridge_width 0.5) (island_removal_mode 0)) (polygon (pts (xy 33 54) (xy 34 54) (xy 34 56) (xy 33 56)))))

